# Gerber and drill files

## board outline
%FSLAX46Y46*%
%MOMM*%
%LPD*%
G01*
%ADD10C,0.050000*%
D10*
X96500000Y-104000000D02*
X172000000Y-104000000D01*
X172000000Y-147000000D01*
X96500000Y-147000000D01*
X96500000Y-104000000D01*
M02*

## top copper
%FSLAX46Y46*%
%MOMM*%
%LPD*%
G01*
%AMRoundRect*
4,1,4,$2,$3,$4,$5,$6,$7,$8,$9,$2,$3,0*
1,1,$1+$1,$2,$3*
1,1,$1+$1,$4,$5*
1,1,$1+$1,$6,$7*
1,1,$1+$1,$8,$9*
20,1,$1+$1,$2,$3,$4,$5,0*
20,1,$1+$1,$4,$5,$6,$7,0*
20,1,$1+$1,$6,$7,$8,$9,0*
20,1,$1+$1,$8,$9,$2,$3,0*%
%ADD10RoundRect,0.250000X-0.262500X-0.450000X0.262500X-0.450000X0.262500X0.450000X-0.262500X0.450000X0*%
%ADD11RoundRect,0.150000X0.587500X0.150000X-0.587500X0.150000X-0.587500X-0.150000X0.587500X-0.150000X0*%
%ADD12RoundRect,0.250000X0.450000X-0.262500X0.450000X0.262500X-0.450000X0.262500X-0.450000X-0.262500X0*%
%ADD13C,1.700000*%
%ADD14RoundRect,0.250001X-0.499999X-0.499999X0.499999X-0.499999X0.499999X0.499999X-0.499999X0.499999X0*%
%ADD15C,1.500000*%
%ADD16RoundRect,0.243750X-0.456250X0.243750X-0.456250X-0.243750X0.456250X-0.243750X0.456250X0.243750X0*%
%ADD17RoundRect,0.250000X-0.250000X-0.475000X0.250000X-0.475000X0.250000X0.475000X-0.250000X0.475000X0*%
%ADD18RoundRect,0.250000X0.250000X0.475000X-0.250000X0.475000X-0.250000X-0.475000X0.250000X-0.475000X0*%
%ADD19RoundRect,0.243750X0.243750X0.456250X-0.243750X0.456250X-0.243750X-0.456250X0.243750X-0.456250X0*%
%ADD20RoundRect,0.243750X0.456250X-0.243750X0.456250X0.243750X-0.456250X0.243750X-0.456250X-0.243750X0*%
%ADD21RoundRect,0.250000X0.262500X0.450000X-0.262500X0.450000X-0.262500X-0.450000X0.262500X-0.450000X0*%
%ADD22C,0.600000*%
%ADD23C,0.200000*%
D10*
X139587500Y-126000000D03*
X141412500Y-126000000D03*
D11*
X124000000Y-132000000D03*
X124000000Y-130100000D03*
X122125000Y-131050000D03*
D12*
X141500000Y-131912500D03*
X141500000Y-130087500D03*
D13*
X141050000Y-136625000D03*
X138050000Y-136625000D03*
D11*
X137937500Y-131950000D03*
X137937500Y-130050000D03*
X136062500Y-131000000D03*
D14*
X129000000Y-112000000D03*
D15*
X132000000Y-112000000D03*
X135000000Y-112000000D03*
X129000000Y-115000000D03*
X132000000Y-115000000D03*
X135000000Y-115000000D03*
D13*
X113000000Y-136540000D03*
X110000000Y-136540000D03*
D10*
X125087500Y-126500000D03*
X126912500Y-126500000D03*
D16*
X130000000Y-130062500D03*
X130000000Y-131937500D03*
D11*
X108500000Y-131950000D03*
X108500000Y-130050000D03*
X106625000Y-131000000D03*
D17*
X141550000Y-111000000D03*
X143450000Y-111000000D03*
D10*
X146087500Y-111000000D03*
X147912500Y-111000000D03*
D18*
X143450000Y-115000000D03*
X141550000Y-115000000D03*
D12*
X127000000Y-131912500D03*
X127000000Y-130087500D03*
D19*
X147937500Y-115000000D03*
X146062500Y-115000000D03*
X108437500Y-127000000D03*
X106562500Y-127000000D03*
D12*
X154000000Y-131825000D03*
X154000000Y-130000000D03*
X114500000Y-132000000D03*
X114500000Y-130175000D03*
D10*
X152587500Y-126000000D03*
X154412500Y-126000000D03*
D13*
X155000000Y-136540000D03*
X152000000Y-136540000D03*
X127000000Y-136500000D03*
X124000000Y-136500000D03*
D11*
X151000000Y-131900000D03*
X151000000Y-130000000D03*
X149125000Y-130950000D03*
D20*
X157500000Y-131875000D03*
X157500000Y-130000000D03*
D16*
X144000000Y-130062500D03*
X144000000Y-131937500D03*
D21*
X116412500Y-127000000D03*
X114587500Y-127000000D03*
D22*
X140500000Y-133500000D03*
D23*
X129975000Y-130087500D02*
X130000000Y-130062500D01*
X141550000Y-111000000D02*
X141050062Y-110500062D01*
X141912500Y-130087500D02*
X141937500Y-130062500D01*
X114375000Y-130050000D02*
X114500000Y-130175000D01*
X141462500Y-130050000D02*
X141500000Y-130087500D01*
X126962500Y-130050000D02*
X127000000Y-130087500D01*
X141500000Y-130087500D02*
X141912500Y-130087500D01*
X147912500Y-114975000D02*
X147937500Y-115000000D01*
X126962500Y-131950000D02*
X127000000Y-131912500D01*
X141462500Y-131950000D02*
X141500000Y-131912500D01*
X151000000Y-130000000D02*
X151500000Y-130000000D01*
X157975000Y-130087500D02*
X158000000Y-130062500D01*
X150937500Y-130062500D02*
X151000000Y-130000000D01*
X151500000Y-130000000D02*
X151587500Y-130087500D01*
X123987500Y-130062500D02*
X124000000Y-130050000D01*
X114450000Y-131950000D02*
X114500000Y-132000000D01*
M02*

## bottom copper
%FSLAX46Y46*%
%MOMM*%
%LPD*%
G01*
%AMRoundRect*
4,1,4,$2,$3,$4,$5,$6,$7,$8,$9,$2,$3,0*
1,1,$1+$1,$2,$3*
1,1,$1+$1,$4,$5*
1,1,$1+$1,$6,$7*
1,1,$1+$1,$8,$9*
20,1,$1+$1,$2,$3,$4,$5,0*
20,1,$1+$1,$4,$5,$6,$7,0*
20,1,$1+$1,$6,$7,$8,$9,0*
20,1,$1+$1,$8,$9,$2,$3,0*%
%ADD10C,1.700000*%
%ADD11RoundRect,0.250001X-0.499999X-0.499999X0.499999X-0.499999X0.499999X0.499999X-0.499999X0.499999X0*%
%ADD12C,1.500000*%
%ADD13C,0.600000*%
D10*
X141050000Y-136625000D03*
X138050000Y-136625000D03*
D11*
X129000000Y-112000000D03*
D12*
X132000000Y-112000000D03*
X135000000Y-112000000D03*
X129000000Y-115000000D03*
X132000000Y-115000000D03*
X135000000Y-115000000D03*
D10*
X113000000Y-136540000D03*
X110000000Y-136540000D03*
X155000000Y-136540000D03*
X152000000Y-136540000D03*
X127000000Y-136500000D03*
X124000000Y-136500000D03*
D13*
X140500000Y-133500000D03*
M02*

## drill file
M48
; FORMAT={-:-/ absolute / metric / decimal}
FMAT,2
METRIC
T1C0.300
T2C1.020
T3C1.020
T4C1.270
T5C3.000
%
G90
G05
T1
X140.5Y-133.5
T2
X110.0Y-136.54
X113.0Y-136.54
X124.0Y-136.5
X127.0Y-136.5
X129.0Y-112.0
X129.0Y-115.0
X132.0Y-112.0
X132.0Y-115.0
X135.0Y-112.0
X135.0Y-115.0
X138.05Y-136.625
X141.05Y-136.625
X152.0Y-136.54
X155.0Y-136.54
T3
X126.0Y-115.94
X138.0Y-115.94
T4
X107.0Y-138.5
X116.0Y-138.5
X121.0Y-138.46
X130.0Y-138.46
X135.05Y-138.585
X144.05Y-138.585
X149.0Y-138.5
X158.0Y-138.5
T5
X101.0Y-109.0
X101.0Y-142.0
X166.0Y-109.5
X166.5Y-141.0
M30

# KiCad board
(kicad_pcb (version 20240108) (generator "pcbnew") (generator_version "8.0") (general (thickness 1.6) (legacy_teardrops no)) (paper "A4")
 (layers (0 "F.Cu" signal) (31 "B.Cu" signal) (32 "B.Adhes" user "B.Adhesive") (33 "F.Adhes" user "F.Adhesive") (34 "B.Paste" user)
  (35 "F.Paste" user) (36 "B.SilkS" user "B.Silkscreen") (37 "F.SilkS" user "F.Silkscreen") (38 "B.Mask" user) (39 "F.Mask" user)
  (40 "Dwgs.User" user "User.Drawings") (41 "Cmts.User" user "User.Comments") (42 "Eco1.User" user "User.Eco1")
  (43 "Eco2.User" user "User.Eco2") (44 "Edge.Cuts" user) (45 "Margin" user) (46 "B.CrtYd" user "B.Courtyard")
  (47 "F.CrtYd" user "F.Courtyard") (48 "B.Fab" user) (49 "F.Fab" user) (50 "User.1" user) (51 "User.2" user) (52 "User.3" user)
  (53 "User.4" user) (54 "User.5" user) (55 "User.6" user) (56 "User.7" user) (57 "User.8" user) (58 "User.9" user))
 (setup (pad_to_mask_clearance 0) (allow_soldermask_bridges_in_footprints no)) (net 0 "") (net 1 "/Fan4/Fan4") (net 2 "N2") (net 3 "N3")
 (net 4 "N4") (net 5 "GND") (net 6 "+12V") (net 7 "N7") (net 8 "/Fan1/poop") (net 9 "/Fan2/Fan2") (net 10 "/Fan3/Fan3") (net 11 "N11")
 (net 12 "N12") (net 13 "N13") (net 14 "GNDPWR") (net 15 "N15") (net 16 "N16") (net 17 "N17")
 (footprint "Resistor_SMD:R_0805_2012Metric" (layer "F.Cu") (at 140.5 126)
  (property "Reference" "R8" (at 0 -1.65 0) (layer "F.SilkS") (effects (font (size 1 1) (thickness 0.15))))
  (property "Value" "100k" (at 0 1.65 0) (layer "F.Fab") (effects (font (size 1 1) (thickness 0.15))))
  (pad "1" smd roundrect (at -0.9125 0) (size 1.025 1.4) (layers "F.Cu" "F.Paste" "F.Mask") (roundrect_rratio 0.243902) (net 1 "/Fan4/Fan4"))
  (pad "2" smd roundrect (at 0.9125 0) (size 1.025 1.4) (layers "F.Cu" "F.Paste" "F.Mask") (roundrect_rratio 0.243902) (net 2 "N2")))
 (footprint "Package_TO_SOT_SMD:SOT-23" (layer "F.Cu") (at 123.0625 131.05 180)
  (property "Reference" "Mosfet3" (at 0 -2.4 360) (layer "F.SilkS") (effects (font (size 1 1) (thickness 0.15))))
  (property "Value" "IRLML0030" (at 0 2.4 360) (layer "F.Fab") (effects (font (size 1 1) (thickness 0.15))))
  (pad "1" smd roundrect (at -0.9375 -0.95 180) (size 1.475 0.6) (layers "F.Cu" "F.Paste" "F.Mask") (roundrect_rratio 0.25) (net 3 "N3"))
  (pad "2" smd roundrect (at -0.9375 0.95 180) (size 1.475 0.6) (layers "F.Cu" "F.Paste" "F.Mask") (roundrect_rratio 0.25) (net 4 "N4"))
  (pad "3" smd roundrect (at 0.9375 0 180) (size 1.475 0.6) (layers "F.Cu" "F.Paste" "F.Mask") (roundrect_rratio 0.25) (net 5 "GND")))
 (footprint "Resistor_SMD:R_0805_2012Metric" (layer "F.Cu") (at 141.5 131 90)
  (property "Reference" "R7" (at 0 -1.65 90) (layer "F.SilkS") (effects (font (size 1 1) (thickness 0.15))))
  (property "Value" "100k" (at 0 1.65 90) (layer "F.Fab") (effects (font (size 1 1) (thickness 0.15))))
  (pad "1" smd roundrect (at -0.9125 0 90) (size 1.025 1.4) (layers "F.Cu" "F.Paste" "F.Mask") (roundrect_rratio 0.243902) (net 2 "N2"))
  (pad "2" smd roundrect (at 0.9125 0 90) (size 1.025 1.4) (layers "F.Cu" "F.Paste" "F.Mask") (roundrect_rratio 0.243902) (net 5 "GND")))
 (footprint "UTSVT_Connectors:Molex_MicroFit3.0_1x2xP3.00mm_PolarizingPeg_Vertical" (layer "F.Cu") (at 141.05 136.625 180)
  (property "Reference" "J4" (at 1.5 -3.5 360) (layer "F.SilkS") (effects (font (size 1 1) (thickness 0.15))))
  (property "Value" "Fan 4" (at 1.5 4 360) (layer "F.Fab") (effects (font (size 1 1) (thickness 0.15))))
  (pad "" np_thru_hole circle (at -3 -1.96 180) (size 1.27 1.27) (drill 1.27) (layers "*.Cu" "*.Mask"))
  (pad "" np_thru_hole circle (at 6 -1.96 180) (size 1.27 1.27) (drill 1.27) (layers "*.Cu" "*.Mask"))
  (pad "1" thru_hole circle (at 0 0 180) (size 1.7 1.7) (drill 1.02) (layers "*.Cu" "*.Mask") (remove_unused_layers no) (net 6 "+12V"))
  (pad "2" thru_hole circle (at 3 0 180) (size 1.7 1.7) (drill 1.02) (layers "*.Cu" "*.Mask") (remove_unused_layers no) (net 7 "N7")))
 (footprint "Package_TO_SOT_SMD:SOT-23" (layer "F.Cu") (at 137 131 180)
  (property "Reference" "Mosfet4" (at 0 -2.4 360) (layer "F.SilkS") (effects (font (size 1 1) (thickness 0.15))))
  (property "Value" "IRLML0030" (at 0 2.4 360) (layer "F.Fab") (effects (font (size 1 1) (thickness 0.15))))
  (pad "1" smd roundrect (at -0.9375 -0.95 180) (size 1.475 0.6) (layers "F.Cu" "F.Paste" "F.Mask") (roundrect_rratio 0.25) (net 2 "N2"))
  (pad "2" smd roundrect (at -0.9375 0.95 180) (size 1.475 0.6) (layers "F.Cu" "F.Paste" "F.Mask") (roundrect_rratio 0.25) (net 7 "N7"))
  (pad "3" smd roundrect (at 0.9375 0 180) (size 1.475 0.6) (layers "F.Cu" "F.Paste" "F.Mask") (roundrect_rratio 0.25) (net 5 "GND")))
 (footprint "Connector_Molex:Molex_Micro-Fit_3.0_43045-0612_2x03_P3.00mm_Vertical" (layer "F.Cu") (at 129 112)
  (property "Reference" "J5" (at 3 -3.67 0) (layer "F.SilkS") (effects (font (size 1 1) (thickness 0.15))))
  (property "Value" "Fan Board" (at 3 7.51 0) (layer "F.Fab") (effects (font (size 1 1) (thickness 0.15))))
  (pad "" np_thru_hole circle (at -3 3.94) (size 1.02 1.02) (drill 1.02) (layers "*.Cu" "*.Mask"))
  (pad "" np_thru_hole circle (at 9 3.94) (size 1.02 1.02) (drill 1.02) (layers "*.Cu" "*.Mask"))
  (pad "1" thru_hole roundrect (at 0 0) (size 1.5 1.5) (drill 1.02) (layers "*.Cu" "*.Mask") (remove_unused_layers no)
   (roundrect_rratio 0.166667) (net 6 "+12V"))
  (pad "2" thru_hole circle (at 3 0) (size 1.5 1.5) (drill 1.02) (layers "*.Cu" "*.Mask") (remove_unused_layers no) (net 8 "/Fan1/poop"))
  (pad "3" thru_hole circle (at 6 0) (size 1.5 1.5) (drill 1.02) (layers "*.Cu" "*.Mask") (remove_unused_layers no) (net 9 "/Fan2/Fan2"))
  (pad "4" thru_hole circle (at 0 3) (size 1.5 1.5) (drill 1.02) (layers "*.Cu" "*.Mask") (remove_unused_layers no) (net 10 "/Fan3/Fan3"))
  (pad "5" thru_hole circle (at 3 3) (size 1.5 1.5) (drill 1.02) (layers "*.Cu" "*.Mask") (remove_unused_layers no) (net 1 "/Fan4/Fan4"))
  (pad "6" thru_hole circle (at 6 3) (size 1.5 1.5) (drill 1.02) (layers "*.Cu" "*.Mask") (remove_unused_layers no) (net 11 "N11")))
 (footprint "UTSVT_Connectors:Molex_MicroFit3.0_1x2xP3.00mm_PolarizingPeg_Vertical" (layer "F.Cu") (at 113 136.54 180)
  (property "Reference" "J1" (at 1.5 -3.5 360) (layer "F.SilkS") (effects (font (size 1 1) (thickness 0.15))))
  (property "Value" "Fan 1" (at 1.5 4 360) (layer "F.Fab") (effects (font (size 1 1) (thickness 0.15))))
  (pad "" np_thru_hole circle (at -3 -1.96 180) (size 1.27 1.27) (drill 1.27) (layers "*.Cu" "*.Mask"))
  (pad "" np_thru_hole circle (at 6 -1.96 180) (size 1.27 1.27) (drill 1.27) (layers "*.Cu" "*.Mask"))
  (pad "1" thru_hole circle (at 0 0 180) (size 1.7 1.7) (drill 1.02) (layers "*.Cu" "*.Mask") (remove_unused_layers no) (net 6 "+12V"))
  (pad "2" thru_hole circle (at 3 0 180) (size 1.7 1.7) (drill 1.02) (layers "*.Cu" "*.Mask") (remove_unused_layers no) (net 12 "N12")))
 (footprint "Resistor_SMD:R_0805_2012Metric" (layer "F.Cu") (at 126 126.5)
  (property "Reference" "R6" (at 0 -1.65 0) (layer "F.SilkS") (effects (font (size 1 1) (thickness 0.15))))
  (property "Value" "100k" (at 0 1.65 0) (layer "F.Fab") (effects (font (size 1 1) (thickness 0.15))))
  (pad "1" smd roundrect (at -0.9125 0) (size 1.025 1.4) (layers "F.Cu" "F.Paste" "F.Mask") (roundrect_rratio 0.243902)
   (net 10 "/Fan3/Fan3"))
  (pad "2" smd roundrect (at 0.9125 0) (size 1.025 1.4) (layers "F.Cu" "F.Paste" "F.Mask") (roundrect_rratio 0.243902) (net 3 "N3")))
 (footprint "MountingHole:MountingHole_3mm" (layer "F.Cu") (at 101 109)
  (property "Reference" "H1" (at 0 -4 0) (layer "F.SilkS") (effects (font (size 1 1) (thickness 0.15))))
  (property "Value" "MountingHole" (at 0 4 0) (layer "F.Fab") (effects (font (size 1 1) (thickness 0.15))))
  (pad "" np_thru_hole circle (at 0 0) (size 3 3) (drill 3) (layers "*.Cu" "*.Mask")))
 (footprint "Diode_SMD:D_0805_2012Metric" (layer "F.Cu") (at 130 131 -90)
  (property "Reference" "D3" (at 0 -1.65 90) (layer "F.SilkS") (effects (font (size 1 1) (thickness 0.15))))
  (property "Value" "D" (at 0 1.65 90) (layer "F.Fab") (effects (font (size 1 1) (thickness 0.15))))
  (pad "1" smd roundrect (at -0.9375 0 270) (size 0.975 1.4) (layers "F.Cu" "F.Paste" "F.Mask") (roundrect_rratio 0.25) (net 6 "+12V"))
  (pad "2" smd roundrect (at 0.9375 0 270) (size 0.975 1.4) (layers "F.Cu" "F.Paste" "F.Mask") (roundrect_rratio 0.25) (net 4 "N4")))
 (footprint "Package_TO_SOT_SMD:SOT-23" (layer "F.Cu") (at 107.5625 131 180)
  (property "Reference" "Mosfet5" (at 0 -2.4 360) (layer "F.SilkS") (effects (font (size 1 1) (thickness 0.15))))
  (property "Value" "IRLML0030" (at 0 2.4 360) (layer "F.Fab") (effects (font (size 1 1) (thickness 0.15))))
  (pad "1" smd roundrect (at -0.9375 -0.95 180) (size 1.475 0.6) (layers "F.Cu" "F.Paste" "F.Mask") (roundrect_rratio 0.25) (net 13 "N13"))
  (pad "2" smd roundrect (at -0.9375 0.95 180) (size 1.475 0.6) (layers "F.Cu" "F.Paste" "F.Mask") (roundrect_rratio 0.25) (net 5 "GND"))
  (pad "3" smd roundrect (at 0.9375 0 180) (size 1.475 0.6) (layers "F.Cu" "F.Paste" "F.Mask") (roundrect_rratio 0.25) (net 12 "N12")))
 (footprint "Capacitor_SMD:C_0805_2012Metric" (layer "F.Cu") (at 142.5 111)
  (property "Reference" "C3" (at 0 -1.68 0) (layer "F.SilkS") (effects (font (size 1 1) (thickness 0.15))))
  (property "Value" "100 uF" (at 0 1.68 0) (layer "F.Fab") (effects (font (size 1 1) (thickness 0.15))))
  (pad "1" smd roundrect (at -0.95 0) (size 1 1.45) (layers "F.Cu" "F.Paste" "F.Mask") (roundrect_rratio 0.25) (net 6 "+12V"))
  (pad "2" smd roundrect (at 0.95 0) (size 1 1.45) (layers "F.Cu" "F.Paste" "F.Mask") (roundrect_rratio 0.25) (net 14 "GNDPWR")))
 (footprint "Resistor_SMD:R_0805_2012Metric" (layer "F.Cu") (at 147 111)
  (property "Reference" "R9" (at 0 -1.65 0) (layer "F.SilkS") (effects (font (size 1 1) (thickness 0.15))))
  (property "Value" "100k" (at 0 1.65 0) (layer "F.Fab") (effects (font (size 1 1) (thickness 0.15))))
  (pad "1" smd roundrect (at -0.9125 0) (size 1.025 1.4) (layers "F.Cu" "F.Paste" "F.Mask") (roundrect_rratio 0.243902) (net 6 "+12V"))
  (pad "2" smd roundrect (at 0.9125 0) (size 1.025 1.4) (layers "F.Cu" "F.Paste" "F.Mask") (roundrect_rratio 0.243902) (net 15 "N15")))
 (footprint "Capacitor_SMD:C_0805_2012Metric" (layer "F.Cu") (at 142.5 115 180)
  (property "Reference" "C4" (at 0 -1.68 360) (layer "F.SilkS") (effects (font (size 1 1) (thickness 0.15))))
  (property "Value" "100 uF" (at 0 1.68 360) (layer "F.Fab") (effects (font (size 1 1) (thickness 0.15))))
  (pad "1" smd roundrect (at -0.95 0 180) (size 1 1.45) (layers "F.Cu" "F.Paste" "F.Mask") (roundrect_rratio 0.25) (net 14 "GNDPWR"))
  (pad "2" smd roundrect (at 0.95 0 180) (size 1 1.45) (layers "F.Cu" "F.Paste" "F.Mask") (roundrect_rratio 0.25) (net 6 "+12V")))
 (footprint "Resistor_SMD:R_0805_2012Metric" (layer "F.Cu") (at 127 131 90)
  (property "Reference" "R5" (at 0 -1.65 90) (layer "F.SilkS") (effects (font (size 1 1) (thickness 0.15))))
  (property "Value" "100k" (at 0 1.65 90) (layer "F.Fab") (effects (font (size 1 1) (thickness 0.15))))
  (pad "1" smd roundrect (at -0.9125 0 90) (size 1.025 1.4) (layers "F.Cu" "F.Paste" "F.Mask") (roundrect_rratio 0.243902) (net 3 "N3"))
  (pad "2" smd roundrect (at 0.9125 0 90) (size 1.025 1.4) (layers "F.Cu" "F.Paste" "F.Mask") (roundrect_rratio 0.243902) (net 5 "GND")))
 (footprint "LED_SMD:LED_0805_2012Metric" (layer "F.Cu") (at 147 115 180)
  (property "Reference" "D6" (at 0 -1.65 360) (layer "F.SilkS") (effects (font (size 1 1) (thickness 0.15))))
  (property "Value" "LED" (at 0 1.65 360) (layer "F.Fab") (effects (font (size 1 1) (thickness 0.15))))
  (pad "1" smd roundrect (at -0.9375 0 180) (size 0.975 1.4) (layers "F.Cu" "F.Paste" "F.Mask") (roundrect_rratio 0.25) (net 15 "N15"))
  (pad "2" smd roundrect (at 0.9375 0 180) (size 0.975 1.4) (layers "F.Cu" "F.Paste" "F.Mask") (roundrect_rratio 0.25) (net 11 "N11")))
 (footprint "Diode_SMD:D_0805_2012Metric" (layer "F.Cu") (at 107.5 127 180)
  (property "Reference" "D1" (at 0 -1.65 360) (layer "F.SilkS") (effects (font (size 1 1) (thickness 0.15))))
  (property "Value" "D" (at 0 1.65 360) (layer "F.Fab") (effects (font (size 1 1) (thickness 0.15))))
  (pad "1" smd roundrect (at -0.9375 0 180) (size 0.975 1.4) (layers "F.Cu" "F.Paste" "F.Mask") (roundrect_rratio 0.25) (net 6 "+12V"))
  (pad "2" smd roundrect (at 0.9375 0 180) (size 0.975 1.4) (layers "F.Cu" "F.Paste" "F.Mask") (roundrect_rratio 0.25) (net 12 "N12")))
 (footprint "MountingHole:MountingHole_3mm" (layer "F.Cu") (at 166 109.5)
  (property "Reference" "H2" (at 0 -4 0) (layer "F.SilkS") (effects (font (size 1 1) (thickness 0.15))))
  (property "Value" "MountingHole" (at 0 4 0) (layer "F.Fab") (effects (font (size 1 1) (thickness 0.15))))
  (pad "" np_thru_hole circle (at 0 0) (size 3 3) (drill 3) (layers "*.Cu" "*.Mask")))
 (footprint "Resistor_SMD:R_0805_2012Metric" (layer "F.Cu") (at 154 130.9125 90)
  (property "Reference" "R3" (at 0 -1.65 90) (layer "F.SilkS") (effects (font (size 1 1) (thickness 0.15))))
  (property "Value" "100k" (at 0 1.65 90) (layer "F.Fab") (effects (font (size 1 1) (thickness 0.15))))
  (pad "1" smd roundrect (at -0.9125 0 90) (size 1.025 1.4) (layers "F.Cu" "F.Paste" "F.Mask") (roundrect_rratio 0.243902) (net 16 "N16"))
  (pad "2" smd roundrect (at 0.9125 0 90) (size 1.025 1.4) (layers "F.Cu" "F.Paste" "F.Mask") (roundrect_rratio 0.243902) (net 5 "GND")))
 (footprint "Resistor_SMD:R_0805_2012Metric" (layer "F.Cu") (at 114.5 131.0875 90)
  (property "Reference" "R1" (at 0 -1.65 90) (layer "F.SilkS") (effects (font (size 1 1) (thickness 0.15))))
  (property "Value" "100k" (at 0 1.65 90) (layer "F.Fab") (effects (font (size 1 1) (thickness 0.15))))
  (pad "1" smd roundrect (at -0.9125 0 90) (size 1.025 1.4) (layers "F.Cu" "F.Paste" "F.Mask") (roundrect_rratio 0.243902) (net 13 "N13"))
  (pad "2" smd roundrect (at 0.9125 0 90) (size 1.025 1.4) (layers "F.Cu" "F.Paste" "F.Mask") (roundrect_rratio 0.243902) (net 5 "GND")))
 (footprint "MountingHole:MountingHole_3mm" (layer "F.Cu") (at 166.5 141)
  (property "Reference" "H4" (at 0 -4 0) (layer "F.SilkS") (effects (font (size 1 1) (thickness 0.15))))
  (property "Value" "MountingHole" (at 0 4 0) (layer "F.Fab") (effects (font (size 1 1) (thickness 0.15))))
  (pad "" np_thru_hole circle (at 0 0) (size 3 3) (drill 3) (layers "*.Cu" "*.Mask")))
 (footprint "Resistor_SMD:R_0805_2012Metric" (layer "F.Cu") (at 153.5 126)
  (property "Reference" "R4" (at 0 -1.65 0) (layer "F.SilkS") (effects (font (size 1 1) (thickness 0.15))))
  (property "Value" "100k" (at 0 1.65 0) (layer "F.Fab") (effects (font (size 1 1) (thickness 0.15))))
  (pad "1" smd roundrect (at -0.9125 0) (size 1.025 1.4) (layers "F.Cu" "F.Paste" "F.Mask") (roundrect_rratio 0.243902) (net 9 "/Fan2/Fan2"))
  (pad "2" smd roundrect (at 0.9125 0) (size 1.025 1.4) (layers "F.Cu" "F.Paste" "F.Mask") (roundrect_rratio 0.243902) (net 16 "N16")))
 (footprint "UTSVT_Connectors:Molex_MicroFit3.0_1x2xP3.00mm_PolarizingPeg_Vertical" (layer "F.Cu") (at 155 136.54 180)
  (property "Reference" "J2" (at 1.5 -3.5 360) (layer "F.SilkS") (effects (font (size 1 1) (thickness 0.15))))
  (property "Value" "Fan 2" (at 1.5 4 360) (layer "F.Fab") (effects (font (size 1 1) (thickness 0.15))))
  (pad "" np_thru_hole circle (at -3 -1.96 180) (size 1.27 1.27) (drill 1.27) (layers "*.Cu" "*.Mask"))
  (pad "" np_thru_hole circle (at 6 -1.96 180) (size 1.27 1.27) (drill 1.27) (layers "*.Cu" "*.Mask"))
  (pad "1" thru_hole circle (at 0 0 180) (size 1.7 1.7) (drill 1.02) (layers "*.Cu" "*.Mask") (remove_unused_layers no) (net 6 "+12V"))
  (pad "2" thru_hole circle (at 3 0 180) (size 1.7 1.7) (drill 1.02) (layers "*.Cu" "*.Mask") (remove_unused_layers no) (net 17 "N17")))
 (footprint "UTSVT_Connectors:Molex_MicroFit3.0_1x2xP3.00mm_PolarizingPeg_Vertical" (layer "F.Cu") (at 127 136.5 180)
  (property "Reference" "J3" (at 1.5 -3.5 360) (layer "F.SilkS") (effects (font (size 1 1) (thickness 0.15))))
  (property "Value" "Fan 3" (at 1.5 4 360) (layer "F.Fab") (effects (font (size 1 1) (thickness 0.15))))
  (pad "" np_thru_hole circle (at -3 -1.96 180) (size 1.27 1.27) (drill 1.27) (layers "*.Cu" "*.Mask"))
  (pad "" np_thru_hole circle (at 6 -1.96 180) (size 1.27 1.27) (drill 1.27) (layers "*.Cu" "*.Mask"))
  (pad "1" thru_hole circle (at 0 0 180) (size 1.7 1.7) (drill 1.02) (layers "*.Cu" "*.Mask") (remove_unused_layers no) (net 6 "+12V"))
  (pad "2" thru_hole circle (at 3 0 180) (size 1.7 1.7) (drill 1.02) (layers "*.Cu" "*.Mask") (remove_unused_layers no) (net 4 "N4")))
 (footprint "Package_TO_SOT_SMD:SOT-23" (layer "F.Cu") (at 150.0625 130.95 180)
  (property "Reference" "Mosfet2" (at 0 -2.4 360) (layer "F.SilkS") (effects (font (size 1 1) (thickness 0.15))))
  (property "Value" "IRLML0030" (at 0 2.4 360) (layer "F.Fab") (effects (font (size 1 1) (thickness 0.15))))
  (pad "1" smd roundrect (at -0.9375 -0.95 180) (size 1.475 0.6) (layers "F.Cu" "F.Paste" "F.Mask") (roundrect_rratio 0.25) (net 16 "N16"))
  (pad "2" smd roundrect (at -0.9375 0.95 180) (size 1.475 0.6) (layers "F.Cu" "F.Paste" "F.Mask") (roundrect_rratio 0.25) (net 17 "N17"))
  (pad "3" smd roundrect (at 0.9375 0 180) (size 1.475 0.6) (layers "F.Cu" "F.Paste" "F.Mask") (roundrect_rratio 0.25) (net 5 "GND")))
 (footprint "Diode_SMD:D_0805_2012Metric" (layer "F.Cu") (at 157.5 130.9375 90)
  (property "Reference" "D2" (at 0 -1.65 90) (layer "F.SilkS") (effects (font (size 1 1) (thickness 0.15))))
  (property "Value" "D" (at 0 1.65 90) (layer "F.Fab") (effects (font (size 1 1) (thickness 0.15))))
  (pad "1" smd roundrect (at -0.9375 0 90) (size 0.975 1.4) (layers "F.Cu" "F.Paste" "F.Mask") (roundrect_rratio 0.25) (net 6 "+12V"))
  (pad "2" smd roundrect (at 0.9375 0 90) (size 0.975 1.4) (layers "F.Cu" "F.Paste" "F.Mask") (roundrect_rratio 0.25) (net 17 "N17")))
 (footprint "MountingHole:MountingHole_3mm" (layer "F.Cu") (at 101 142)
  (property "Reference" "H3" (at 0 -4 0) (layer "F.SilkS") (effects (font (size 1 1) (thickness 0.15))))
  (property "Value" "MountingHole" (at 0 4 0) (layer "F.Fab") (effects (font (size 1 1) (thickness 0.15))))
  (pad "" np_thru_hole circle (at 0 0) (size 3 3) (drill 3) (layers "*.Cu" "*.Mask")))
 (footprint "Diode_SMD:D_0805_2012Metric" (layer "F.Cu") (at 144 131 -90)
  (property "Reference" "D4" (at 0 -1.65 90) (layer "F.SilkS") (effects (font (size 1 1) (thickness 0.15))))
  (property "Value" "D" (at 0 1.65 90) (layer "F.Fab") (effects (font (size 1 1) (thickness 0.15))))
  (pad "1" smd roundrect (at -0.9375 0 270) (size 0.975 1.4) (layers "F.Cu" "F.Paste" "F.Mask") (roundrect_rratio 0.25) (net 6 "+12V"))
  (pad "2" smd roundrect (at 0.9375 0 270) (size 0.975 1.4) (layers "F.Cu" "F.Paste" "F.Mask") (roundrect_rratio 0.25) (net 7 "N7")))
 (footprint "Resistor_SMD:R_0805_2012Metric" (layer "F.Cu") (at 115.5 127 180)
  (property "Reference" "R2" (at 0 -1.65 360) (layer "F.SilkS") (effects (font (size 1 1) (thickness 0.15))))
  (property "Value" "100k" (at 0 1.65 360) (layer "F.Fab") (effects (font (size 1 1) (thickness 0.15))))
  (pad "1" smd roundrect (at -0.9125 0 180) (size 1.025 1.4) (layers "F.Cu" "F.Paste" "F.Mask") (roundrect_rratio 0.243902)
   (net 8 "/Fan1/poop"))
  (pad "2" smd roundrect (at 0.9125 0 180) (size 1.025 1.4) (layers "F.Cu" "F.Paste" "F.Mask") (roundrect_rratio 0.243902) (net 13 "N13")))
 (gr_rect (start 96.5 104) (end 172 147) (stroke (width 0.05) (type default)) (fill none) (layer "Edge.Cuts"))
 (segment (start 129.975 130.0875) (end 130 130.0625) (width 0.2) (layer "F.Cu") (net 6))
 (segment (start 141.55 111) (end 141.050062 110.500062) (width 0.2) (layer "F.Cu") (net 6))
 (segment (start 141.9125 130.0875) (end 141.9375 130.0625) (width 0.2) (layer "F.Cu") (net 5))
 (segment (start 114.375 130.05) (end 114.5 130.175) (width 0.2) (layer "F.Cu") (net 5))
 (segment (start 141.4625 130.05) (end 141.5 130.0875) (width 0.2) (layer "F.Cu") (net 5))
 (segment (start 126.9625 130.05) (end 127 130.0875) (width 0.2) (layer "F.Cu") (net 5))
 (segment (start 141.5 130.0875) (end 141.9125 130.0875) (width 0.2) (layer "F.Cu") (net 5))
 (segment (start 147.9125 114.975) (end 147.9375 115) (width 0.2) (layer "F.Cu") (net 15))
 (segment (start 126.9625 131.95) (end 127 131.9125) (width 0.2) (layer "F.Cu") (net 3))
 (segment (start 141.4625 131.95) (end 141.5 131.9125) (width 0.2) (layer "F.Cu") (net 2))
 (via (at 140.5 133.5) (size 0.6) (drill 0.3) (layers "F.Cu" "B.Cu") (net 2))
 (segment (start 151 130) (end 151.5 130) (width 0.2) (layer "F.Cu") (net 17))
 (segment (start 157.975 130.0875) (end 158 130.0625) (width 0.2) (layer "F.Cu") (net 17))
 (segment (start 150.9375 130.0625) (end 151 130) (width 0.2) (layer "F.Cu") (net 17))
 (segment (start 151.5 130) (end 151.5875 130.0875) (width 0.2) (layer "F.Cu") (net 17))
 (segment (start 123.9875 130.0625) (end 124 130.05) (width 0.2) (layer "F.Cu") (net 4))
 (segment (start 114.45 131.95) (end 114.5 132) (width 0.2) (layer "F.Cu") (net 13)))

